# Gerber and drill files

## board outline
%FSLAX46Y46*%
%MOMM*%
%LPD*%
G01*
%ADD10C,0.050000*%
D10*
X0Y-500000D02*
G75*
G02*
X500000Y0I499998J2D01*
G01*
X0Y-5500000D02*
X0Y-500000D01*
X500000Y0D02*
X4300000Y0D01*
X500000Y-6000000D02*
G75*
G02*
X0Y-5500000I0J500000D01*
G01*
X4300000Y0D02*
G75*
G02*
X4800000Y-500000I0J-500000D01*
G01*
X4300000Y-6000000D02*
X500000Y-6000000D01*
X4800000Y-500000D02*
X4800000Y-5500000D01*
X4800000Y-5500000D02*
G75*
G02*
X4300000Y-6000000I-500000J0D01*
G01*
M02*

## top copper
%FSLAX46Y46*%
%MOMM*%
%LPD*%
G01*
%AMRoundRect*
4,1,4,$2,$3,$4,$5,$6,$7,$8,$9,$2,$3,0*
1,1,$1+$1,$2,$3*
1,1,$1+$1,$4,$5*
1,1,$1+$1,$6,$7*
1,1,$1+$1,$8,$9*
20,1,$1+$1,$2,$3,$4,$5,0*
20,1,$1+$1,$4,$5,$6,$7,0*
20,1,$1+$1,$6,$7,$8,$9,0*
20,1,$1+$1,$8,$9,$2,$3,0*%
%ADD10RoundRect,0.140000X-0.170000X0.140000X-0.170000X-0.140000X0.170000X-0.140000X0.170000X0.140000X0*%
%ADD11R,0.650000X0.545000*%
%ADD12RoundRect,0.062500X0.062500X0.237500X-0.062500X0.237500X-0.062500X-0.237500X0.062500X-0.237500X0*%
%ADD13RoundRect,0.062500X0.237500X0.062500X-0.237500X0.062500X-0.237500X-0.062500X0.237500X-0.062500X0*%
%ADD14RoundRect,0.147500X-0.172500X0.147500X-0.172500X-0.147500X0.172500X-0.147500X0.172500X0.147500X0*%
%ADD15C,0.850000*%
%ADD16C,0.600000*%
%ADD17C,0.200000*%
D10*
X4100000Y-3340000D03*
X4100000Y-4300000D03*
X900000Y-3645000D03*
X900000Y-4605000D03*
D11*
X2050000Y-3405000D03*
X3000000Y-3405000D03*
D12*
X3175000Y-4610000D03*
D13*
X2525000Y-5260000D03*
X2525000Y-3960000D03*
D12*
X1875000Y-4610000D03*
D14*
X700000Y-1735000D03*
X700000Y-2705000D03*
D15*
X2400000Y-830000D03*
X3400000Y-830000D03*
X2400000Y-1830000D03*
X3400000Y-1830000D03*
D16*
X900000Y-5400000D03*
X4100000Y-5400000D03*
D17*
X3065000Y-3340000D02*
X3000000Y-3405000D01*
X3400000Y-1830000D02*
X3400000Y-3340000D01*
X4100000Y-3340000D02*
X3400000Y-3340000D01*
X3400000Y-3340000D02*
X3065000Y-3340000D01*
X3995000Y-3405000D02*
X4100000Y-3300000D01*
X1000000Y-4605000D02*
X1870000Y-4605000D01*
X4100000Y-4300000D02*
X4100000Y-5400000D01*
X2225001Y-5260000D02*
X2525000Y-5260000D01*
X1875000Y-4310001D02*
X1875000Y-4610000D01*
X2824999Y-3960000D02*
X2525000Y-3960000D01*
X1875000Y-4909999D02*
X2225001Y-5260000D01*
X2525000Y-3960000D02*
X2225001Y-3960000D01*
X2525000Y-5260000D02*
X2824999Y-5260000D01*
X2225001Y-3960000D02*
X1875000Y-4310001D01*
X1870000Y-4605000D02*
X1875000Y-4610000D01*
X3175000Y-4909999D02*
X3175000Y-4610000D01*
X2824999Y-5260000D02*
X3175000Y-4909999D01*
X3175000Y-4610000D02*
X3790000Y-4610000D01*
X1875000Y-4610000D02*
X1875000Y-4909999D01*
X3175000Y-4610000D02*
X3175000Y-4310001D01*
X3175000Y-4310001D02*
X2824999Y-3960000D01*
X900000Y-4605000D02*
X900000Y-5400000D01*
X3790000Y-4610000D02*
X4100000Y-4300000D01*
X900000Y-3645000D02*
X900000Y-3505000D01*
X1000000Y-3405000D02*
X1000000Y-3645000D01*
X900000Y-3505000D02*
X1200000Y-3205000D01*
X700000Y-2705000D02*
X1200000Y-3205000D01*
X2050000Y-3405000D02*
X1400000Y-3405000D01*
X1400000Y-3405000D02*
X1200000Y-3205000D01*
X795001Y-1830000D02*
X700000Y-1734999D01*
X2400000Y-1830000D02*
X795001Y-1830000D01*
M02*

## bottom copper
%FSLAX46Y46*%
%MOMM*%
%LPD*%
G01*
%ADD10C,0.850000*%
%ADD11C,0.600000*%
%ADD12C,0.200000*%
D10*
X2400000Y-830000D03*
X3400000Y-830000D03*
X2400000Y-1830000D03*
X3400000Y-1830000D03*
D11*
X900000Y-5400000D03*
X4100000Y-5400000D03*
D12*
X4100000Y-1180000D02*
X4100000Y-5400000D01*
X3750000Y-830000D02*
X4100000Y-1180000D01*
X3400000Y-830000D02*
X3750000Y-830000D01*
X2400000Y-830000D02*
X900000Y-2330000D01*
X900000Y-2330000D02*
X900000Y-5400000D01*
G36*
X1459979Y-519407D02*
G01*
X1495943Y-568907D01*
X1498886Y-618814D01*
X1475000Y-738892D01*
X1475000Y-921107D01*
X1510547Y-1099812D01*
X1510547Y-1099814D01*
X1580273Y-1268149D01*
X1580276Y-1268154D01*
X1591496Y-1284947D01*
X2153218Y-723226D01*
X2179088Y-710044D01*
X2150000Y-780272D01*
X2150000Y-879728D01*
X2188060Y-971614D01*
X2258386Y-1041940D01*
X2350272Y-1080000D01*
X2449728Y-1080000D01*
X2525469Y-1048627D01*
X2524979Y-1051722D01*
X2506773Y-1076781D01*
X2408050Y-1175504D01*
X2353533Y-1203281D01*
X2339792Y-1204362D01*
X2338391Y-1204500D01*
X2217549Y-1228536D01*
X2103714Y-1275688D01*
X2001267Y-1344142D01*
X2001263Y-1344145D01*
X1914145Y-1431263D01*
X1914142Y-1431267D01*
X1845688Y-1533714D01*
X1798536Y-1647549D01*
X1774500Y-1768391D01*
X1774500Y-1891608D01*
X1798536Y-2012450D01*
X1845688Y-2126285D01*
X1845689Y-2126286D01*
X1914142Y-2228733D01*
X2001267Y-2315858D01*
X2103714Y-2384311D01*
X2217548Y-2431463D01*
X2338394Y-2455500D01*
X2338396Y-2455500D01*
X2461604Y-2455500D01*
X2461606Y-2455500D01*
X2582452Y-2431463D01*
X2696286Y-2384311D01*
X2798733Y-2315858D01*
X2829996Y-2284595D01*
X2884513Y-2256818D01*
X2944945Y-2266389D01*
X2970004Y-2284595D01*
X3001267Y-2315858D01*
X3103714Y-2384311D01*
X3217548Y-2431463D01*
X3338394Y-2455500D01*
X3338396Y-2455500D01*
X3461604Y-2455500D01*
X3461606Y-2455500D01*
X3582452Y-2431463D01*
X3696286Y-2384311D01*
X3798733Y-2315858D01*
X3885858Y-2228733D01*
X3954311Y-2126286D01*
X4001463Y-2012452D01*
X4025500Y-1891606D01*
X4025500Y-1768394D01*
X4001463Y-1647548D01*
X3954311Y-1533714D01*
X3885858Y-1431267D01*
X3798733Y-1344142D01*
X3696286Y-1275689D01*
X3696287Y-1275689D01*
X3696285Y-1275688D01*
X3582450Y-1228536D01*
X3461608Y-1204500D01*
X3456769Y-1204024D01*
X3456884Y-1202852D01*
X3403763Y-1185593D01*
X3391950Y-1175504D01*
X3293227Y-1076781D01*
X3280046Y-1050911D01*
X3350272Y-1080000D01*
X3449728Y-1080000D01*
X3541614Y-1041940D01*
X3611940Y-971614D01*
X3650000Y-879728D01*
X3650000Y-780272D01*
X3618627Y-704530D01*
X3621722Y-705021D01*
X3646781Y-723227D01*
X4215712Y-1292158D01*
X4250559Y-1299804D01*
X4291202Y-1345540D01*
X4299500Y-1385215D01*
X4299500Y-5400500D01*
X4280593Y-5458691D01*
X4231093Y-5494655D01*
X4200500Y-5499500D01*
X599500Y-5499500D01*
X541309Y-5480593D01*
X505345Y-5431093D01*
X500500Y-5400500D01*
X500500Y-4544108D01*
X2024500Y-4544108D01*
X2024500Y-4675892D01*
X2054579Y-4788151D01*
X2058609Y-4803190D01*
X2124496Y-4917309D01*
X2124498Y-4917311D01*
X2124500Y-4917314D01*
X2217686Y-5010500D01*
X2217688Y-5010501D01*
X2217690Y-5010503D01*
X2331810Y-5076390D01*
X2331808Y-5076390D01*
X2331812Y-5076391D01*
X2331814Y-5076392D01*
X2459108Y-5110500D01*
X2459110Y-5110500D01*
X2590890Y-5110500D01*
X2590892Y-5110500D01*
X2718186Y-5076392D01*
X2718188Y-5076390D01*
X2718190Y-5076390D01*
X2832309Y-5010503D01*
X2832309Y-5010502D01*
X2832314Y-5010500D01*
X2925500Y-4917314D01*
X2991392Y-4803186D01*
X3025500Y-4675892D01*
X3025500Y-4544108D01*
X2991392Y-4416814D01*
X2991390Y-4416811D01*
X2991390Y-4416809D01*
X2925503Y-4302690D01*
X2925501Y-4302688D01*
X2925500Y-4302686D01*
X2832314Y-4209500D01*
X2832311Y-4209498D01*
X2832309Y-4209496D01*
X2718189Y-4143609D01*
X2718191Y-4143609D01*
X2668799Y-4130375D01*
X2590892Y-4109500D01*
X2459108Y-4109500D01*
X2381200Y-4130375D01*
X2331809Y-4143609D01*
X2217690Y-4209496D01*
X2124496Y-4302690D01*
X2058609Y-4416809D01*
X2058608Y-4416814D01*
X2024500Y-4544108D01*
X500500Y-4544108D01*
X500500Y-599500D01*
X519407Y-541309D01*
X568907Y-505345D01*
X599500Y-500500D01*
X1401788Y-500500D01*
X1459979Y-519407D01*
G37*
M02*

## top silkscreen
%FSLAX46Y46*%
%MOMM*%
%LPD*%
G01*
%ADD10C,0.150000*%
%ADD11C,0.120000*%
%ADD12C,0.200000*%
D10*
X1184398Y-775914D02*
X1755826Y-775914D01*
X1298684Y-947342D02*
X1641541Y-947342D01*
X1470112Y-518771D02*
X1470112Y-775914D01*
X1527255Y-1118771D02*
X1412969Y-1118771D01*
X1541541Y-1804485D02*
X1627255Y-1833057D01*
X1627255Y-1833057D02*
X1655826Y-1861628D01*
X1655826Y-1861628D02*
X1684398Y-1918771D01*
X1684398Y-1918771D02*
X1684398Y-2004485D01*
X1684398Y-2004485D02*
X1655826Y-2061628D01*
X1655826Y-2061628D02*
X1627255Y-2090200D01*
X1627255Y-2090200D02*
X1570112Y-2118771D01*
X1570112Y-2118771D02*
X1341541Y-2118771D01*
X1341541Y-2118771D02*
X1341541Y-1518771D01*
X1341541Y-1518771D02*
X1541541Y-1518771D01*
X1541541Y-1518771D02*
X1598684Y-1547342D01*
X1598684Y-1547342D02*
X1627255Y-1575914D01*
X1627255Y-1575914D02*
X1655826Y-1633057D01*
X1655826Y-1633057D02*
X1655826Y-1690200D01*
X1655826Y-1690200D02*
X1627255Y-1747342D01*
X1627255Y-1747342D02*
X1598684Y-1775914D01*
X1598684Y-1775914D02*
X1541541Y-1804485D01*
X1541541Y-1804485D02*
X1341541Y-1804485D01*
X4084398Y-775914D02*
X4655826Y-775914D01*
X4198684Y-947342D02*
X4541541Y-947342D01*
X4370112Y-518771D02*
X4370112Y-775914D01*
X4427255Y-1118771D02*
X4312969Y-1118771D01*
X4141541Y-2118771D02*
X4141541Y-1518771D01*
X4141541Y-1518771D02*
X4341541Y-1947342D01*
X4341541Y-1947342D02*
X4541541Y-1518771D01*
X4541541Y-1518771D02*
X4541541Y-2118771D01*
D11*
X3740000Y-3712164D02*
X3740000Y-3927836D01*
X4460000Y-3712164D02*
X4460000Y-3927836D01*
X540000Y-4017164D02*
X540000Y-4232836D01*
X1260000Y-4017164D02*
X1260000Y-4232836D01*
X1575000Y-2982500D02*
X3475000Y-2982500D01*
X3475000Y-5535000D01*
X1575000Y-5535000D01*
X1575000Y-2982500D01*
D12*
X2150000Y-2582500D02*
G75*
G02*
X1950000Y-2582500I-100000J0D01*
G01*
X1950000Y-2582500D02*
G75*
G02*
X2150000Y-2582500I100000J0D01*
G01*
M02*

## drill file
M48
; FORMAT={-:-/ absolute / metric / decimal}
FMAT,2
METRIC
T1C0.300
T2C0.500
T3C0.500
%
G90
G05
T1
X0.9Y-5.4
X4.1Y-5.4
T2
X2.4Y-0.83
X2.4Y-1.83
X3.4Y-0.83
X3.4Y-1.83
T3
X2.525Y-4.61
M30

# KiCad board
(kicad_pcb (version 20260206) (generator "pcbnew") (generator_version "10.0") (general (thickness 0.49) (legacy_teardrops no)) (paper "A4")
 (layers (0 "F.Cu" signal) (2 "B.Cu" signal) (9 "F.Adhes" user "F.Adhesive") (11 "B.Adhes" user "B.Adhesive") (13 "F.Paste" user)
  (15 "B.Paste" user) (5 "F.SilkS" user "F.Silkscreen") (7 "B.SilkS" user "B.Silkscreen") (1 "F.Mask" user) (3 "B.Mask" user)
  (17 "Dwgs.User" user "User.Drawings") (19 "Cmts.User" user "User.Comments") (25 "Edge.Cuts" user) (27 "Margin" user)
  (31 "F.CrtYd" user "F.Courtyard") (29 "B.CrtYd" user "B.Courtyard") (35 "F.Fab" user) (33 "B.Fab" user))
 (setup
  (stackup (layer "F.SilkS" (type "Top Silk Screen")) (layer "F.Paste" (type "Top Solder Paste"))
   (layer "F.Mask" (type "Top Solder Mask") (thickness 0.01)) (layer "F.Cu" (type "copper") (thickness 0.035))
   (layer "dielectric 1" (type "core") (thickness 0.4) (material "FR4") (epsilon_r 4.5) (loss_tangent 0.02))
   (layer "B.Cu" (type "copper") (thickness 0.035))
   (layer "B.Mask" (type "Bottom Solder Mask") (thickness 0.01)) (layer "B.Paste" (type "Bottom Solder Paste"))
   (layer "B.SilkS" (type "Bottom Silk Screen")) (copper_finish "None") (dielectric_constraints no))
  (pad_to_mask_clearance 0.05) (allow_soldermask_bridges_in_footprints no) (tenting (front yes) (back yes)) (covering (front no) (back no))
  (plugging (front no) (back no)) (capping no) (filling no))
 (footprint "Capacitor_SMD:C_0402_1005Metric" (layer "F.Cu") (at 4.1 3.82 -90)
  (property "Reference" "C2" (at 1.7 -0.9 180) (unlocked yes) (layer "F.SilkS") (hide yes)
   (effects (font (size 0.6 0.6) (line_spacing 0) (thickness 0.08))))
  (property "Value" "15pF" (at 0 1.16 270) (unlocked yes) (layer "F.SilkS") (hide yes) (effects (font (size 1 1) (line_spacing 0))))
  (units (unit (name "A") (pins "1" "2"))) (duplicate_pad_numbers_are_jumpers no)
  (fp_line (start -0.107836 0.36) (end 0.107836 0.36) (stroke (width 0.12) (type solid)) (layer "F.SilkS"))
  (fp_line (start -0.107836 -0.36) (end 0.107836 -0.36) (stroke (width 0.12) (type solid)) (layer "F.SilkS"))
  (pad "1" smd roundrect (at -0.48 0 270) (size 0.56 0.62) (layers "F.Cu" "F.Mask" "F.Paste") (roundrect_rratio 0.25) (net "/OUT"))
  (pad "2" smd roundrect (at 0.48 0 270) (size 0.56 0.62) (layers "F.Cu" "F.Mask" "F.Paste") (roundrect_rratio 0.25) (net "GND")))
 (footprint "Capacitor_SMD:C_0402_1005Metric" (layer "F.Cu") (at 0.9 4.125 -90)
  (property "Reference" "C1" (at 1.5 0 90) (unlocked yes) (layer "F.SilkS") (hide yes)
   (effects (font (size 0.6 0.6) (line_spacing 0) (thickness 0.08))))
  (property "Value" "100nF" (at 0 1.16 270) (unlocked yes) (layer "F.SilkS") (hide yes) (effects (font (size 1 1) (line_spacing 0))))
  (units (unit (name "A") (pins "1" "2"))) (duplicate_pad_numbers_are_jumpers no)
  (fp_line (start -0.107836 0.36) (end 0.107836 0.36) (stroke (width 0.12) (type solid)) (layer "F.SilkS"))
  (fp_line (start -0.107836 -0.36) (end 0.107836 -0.36) (stroke (width 0.12) (type solid)) (layer "F.SilkS"))
  (pad "1" smd roundrect (at -0.48 0 270) (size 0.56 0.62) (layers "F.Cu" "F.Mask" "F.Paste") (roundrect_rratio 0.25) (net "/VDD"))
  (pad "2" smd roundrect (at 0.48 0 270) (size 0.56 0.62) (layers "F.Cu" "F.Mask" "F.Paste") (roundrect_rratio 0.25) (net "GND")))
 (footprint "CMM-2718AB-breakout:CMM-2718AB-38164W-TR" (layer "F.Cu") (at 2.525 4.61 180)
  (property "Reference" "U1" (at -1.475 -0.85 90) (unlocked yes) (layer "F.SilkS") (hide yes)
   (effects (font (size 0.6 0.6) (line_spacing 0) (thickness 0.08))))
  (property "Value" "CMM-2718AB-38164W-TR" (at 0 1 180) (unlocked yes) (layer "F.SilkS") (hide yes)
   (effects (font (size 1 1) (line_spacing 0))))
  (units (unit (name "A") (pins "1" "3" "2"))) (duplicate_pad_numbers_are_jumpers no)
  (fp_rect (start 0.95 1.6275) (end -0.95 -0.925) (stroke (width 0.12) (type default)) (fill no) (layer "F.SilkS"))
  (fp_circle (center 0.475 2.0275) (end 0.325 2.0275) (stroke (width 0.1) (type default)) (fill yes) (layer "F.SilkS"))
  (pad "" np_thru_hole circle (at 0 0 180) (size 0.5 0.5) (drill 0.5) (layers "*.Cu" "*.Mask"))
  (pad "1" smd rect (at 0.475 1.205 180) (size 0.65 0.545) (layers "F.Cu" "F.Mask" "F.Paste") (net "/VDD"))
  (pad "2" smd rect (at -0.475 1.205 180) (size 0.65 0.545) (layers "F.Cu" "F.Mask" "F.Paste") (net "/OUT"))
  (pad "3" smd roundrect (at -0.65 0 180) (size 0.25 0.6) (layers "F.Cu" "F.Mask" "F.Paste") (roundrect_rratio 0.25) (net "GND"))
  (pad "3" smd roundrect (at 0 -0.65 180) (size 0.6 0.25) (layers "F.Cu" "F.Mask" "F.Paste") (roundrect_rratio 0.25) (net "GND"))
  (pad "3" smd roundrect (at 0 0.65 180) (size 0.6 0.25) (layers "F.Cu" "F.Mask" "F.Paste") (roundrect_rratio 0.25) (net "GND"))
  (pad "3" smd roundrect (at 0.65 0 180) (size 0.25 0.6) (layers "F.Cu" "F.Mask" "F.Paste") (roundrect_rratio 0.25) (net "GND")))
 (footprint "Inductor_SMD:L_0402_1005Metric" (layer "F.Cu") (at 0.7 2.22 -90)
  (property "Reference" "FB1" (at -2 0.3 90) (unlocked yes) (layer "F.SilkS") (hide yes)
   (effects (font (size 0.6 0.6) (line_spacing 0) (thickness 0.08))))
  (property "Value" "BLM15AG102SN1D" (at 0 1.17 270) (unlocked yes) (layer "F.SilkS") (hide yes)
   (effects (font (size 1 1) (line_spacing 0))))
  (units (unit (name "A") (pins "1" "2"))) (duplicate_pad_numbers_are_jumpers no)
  (pad "1" smd roundrect (at -0.485 0 270) (size 0.59 0.64) (layers "F.Cu" "F.Mask" "F.Paste") (roundrect_rratio 0.25) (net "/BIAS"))
  (pad "2" smd roundrect (at 0.485 0 270) (size 0.59 0.64) (layers "F.Cu" "F.Mask" "F.Paste") (roundrect_rratio 0.25) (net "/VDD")))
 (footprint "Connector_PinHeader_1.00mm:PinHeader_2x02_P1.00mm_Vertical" (layer "F.Cu") (at 2.4 0.83)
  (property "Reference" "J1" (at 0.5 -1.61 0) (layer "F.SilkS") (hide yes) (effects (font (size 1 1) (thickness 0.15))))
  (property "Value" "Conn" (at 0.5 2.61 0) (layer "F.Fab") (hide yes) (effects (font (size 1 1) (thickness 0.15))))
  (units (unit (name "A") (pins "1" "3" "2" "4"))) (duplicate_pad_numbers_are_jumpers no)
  (pad "1" thru_hole circle (at 0 0) (size 0.85 0.85) (drill 0.5) (layers "*.Cu" "*.Mask") (remove_unused_layers no) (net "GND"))
  (pad "2" thru_hole circle (at 1 0) (size 0.85 0.85) (drill 0.5) (layers "*.Cu" "*.Mask") (remove_unused_layers no) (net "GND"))
  (pad "3" thru_hole circle (at 0 1) (size 0.85 0.85) (drill 0.5) (layers "*.Cu" "*.Mask") (remove_unused_layers no) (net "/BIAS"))
  (pad "4" thru_hole circle (at 1 1) (size 0.85 0.85) (drill 0.5) (layers "*.Cu" "*.Mask") (remove_unused_layers no) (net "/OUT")))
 (gr_arc (start 0 0.5) (mid 0.146446 0.146446) (end 0.5 0) (stroke (width 0.05) (type default)) (layer "Edge.Cuts"))
 (gr_line (start 0 5.5) (end 0 0.5) (stroke (width 0.05) (type default)) (layer "Edge.Cuts"))
 (gr_line (start 0.5 0) (end 4.3 0) (stroke (width 0.05) (type default)) (layer "Edge.Cuts"))
 (gr_arc (start 0.5 6) (mid 0.146447 5.853553) (end 0 5.5) (stroke (width 0.05) (type default)) (layer "Edge.Cuts"))
 (gr_arc (start 4.3 0) (mid 4.653553 0.146447) (end 4.8 0.5) (stroke (width 0.05) (type default)) (layer "Edge.Cuts"))
 (gr_line (start 4.3 6) (end 0.5 6) (stroke (width 0.05) (type default)) (layer "Edge.Cuts"))
 (gr_line (start 4.8 0.5) (end 4.8 5.5) (stroke (width 0.05) (type default)) (layer "Edge.Cuts"))
 (gr_arc (start 4.8 5.5) (mid 4.653553 5.853553) (end 4.3 6) (stroke (width 0.05) (type default)) (layer "Edge.Cuts"))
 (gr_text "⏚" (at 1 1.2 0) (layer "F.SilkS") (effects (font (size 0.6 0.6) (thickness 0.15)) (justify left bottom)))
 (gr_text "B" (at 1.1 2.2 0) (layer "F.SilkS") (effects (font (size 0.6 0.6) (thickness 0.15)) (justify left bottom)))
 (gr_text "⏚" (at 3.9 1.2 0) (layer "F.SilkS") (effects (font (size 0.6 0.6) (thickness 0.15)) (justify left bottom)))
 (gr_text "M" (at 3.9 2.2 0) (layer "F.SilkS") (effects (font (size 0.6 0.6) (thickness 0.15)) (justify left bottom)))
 (segment (start 3.065 3.34) (end 3 3.405) (width 0.2) (layer "F.Cu") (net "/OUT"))
 (segment (start 3.4 1.83) (end 3.4 3.34) (width 0.2) (layer "F.Cu") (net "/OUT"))
 (segment (start 4.1 3.34) (end 3.4 3.34) (width 0.2) (layer "F.Cu") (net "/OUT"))
 (segment (start 3.4 3.34) (end 3.065 3.34) (width 0.2) (layer "F.Cu") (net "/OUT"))
 (segment (start 3.995 3.405) (end 4.1 3.3) (width 0.2) (layer "F.Cu") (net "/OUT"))
 (segment (start 1 4.605) (end 1.87 4.605) (width 0.2) (layer "F.Cu") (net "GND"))
 (segment (start 4.1 4.3) (end 4.1 5.4) (width 0.2) (layer "F.Cu") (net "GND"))
 (segment (start 2.225001 5.26) (end 2.525 5.26) (width 0.2) (layer "F.Cu") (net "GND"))
 (segment (start 1.875 4.310001) (end 1.875 4.61) (width 0.2) (layer "F.Cu") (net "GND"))
 (segment (start 2.824999 3.96) (end 2.525 3.96) (width 0.2) (layer "F.Cu") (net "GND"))
 (segment (start 1.875 4.909999) (end 2.225001 5.26) (width 0.2) (layer "F.Cu") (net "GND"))
 (segment (start 2.525 3.96) (end 2.225001 3.96) (width 0.2) (layer "F.Cu") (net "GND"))
 (segment (start 2.525 5.26) (end 2.824999 5.26) (width 0.2) (layer "F.Cu") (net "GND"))
 (segment (start 2.225001 3.96) (end 1.875 4.310001) (width 0.2) (layer "F.Cu") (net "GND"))
 (segment (start 1.87 4.605) (end 1.875 4.61) (width 0.2) (layer "F.Cu") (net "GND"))
 (segment (start 3.175 4.909999) (end 3.175 4.61) (width 0.2) (layer "F.Cu") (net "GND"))
 (segment (start 2.824999 5.26) (end 3.175 4.909999) (width 0.2) (layer "F.Cu") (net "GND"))
 (segment (start 3.175 4.61) (end 3.79 4.61) (width 0.2) (layer "F.Cu") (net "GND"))
 (segment (start 1.875 4.61) (end 1.875 4.909999) (width 0.2) (layer "F.Cu") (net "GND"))
 (segment (start 3.175 4.61) (end 3.175 4.310001) (width 0.2) (layer "F.Cu") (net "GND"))
 (segment (start 3.175 4.310001) (end 2.824999 3.96) (width 0.2) (layer "F.Cu") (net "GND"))
 (segment (start 0.9 4.605) (end 0.9 5.4) (width 0.2) (layer "F.Cu") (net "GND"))
 (segment (start 3.79 4.61) (end 4.1 4.3) (width 0.2) (layer "F.Cu") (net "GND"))
 (via (at 0.9 5.4) (size 0.6) (drill 0.3) (layers "F.Cu" "B.Cu") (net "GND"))
 (via (at 4.1 5.4) (size 0.6) (drill 0.3) (layers "F.Cu" "B.Cu") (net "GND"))
 (segment (start 4.1 1.18) (end 4.1 5.4) (width 0.2) (layer "B.Cu") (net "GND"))
 (segment (start 3.75 0.83) (end 4.1 1.18) (width 0.2) (layer "B.Cu") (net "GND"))
 (segment (start 3.4 0.83) (end 3.75 0.83) (width 0.2) (layer "B.Cu") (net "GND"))
 (segment (start 2.4 0.83) (end 0.9 2.33) (width 0.2) (layer "B.Cu") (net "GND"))
 (segment (start 0.9 2.33) (end 0.9 5.4) (width 0.2) (layer "B.Cu") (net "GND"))
 (segment (start 0.9 3.645) (end 0.9 3.505) (width 0.2) (layer "F.Cu") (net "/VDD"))
 (segment (start 1 3.405) (end 1 3.645) (width 0.2) (layer "F.Cu") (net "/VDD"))
 (segment (start 0.9 3.505) (end 1.2 3.205) (width 0.2) (layer "F.Cu") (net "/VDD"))
 (segment (start 0.7 2.705) (end 1.2 3.205) (width 0.2) (layer "F.Cu") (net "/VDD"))
 (segment (start 2.05 3.405) (end 1.4 3.405) (width 0.2) (layer "F.Cu") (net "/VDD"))
 (segment (start 1.4 3.405) (end 1.2 3.205) (width 0.2) (layer "F.Cu") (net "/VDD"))
 (segment (start 0.795001 1.83) (end 0.7 1.734999) (width 0.2) (layer "F.Cu") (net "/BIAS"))
 (segment (start 2.4 1.83) (end 0.795001 1.83) (width 0.2) (layer "F.Cu") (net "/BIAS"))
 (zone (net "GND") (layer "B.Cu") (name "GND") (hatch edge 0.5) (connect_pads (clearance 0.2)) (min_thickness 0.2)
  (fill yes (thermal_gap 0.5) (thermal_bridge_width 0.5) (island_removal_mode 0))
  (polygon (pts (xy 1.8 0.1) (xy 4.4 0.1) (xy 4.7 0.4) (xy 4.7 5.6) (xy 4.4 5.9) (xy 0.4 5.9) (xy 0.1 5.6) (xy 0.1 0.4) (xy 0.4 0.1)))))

